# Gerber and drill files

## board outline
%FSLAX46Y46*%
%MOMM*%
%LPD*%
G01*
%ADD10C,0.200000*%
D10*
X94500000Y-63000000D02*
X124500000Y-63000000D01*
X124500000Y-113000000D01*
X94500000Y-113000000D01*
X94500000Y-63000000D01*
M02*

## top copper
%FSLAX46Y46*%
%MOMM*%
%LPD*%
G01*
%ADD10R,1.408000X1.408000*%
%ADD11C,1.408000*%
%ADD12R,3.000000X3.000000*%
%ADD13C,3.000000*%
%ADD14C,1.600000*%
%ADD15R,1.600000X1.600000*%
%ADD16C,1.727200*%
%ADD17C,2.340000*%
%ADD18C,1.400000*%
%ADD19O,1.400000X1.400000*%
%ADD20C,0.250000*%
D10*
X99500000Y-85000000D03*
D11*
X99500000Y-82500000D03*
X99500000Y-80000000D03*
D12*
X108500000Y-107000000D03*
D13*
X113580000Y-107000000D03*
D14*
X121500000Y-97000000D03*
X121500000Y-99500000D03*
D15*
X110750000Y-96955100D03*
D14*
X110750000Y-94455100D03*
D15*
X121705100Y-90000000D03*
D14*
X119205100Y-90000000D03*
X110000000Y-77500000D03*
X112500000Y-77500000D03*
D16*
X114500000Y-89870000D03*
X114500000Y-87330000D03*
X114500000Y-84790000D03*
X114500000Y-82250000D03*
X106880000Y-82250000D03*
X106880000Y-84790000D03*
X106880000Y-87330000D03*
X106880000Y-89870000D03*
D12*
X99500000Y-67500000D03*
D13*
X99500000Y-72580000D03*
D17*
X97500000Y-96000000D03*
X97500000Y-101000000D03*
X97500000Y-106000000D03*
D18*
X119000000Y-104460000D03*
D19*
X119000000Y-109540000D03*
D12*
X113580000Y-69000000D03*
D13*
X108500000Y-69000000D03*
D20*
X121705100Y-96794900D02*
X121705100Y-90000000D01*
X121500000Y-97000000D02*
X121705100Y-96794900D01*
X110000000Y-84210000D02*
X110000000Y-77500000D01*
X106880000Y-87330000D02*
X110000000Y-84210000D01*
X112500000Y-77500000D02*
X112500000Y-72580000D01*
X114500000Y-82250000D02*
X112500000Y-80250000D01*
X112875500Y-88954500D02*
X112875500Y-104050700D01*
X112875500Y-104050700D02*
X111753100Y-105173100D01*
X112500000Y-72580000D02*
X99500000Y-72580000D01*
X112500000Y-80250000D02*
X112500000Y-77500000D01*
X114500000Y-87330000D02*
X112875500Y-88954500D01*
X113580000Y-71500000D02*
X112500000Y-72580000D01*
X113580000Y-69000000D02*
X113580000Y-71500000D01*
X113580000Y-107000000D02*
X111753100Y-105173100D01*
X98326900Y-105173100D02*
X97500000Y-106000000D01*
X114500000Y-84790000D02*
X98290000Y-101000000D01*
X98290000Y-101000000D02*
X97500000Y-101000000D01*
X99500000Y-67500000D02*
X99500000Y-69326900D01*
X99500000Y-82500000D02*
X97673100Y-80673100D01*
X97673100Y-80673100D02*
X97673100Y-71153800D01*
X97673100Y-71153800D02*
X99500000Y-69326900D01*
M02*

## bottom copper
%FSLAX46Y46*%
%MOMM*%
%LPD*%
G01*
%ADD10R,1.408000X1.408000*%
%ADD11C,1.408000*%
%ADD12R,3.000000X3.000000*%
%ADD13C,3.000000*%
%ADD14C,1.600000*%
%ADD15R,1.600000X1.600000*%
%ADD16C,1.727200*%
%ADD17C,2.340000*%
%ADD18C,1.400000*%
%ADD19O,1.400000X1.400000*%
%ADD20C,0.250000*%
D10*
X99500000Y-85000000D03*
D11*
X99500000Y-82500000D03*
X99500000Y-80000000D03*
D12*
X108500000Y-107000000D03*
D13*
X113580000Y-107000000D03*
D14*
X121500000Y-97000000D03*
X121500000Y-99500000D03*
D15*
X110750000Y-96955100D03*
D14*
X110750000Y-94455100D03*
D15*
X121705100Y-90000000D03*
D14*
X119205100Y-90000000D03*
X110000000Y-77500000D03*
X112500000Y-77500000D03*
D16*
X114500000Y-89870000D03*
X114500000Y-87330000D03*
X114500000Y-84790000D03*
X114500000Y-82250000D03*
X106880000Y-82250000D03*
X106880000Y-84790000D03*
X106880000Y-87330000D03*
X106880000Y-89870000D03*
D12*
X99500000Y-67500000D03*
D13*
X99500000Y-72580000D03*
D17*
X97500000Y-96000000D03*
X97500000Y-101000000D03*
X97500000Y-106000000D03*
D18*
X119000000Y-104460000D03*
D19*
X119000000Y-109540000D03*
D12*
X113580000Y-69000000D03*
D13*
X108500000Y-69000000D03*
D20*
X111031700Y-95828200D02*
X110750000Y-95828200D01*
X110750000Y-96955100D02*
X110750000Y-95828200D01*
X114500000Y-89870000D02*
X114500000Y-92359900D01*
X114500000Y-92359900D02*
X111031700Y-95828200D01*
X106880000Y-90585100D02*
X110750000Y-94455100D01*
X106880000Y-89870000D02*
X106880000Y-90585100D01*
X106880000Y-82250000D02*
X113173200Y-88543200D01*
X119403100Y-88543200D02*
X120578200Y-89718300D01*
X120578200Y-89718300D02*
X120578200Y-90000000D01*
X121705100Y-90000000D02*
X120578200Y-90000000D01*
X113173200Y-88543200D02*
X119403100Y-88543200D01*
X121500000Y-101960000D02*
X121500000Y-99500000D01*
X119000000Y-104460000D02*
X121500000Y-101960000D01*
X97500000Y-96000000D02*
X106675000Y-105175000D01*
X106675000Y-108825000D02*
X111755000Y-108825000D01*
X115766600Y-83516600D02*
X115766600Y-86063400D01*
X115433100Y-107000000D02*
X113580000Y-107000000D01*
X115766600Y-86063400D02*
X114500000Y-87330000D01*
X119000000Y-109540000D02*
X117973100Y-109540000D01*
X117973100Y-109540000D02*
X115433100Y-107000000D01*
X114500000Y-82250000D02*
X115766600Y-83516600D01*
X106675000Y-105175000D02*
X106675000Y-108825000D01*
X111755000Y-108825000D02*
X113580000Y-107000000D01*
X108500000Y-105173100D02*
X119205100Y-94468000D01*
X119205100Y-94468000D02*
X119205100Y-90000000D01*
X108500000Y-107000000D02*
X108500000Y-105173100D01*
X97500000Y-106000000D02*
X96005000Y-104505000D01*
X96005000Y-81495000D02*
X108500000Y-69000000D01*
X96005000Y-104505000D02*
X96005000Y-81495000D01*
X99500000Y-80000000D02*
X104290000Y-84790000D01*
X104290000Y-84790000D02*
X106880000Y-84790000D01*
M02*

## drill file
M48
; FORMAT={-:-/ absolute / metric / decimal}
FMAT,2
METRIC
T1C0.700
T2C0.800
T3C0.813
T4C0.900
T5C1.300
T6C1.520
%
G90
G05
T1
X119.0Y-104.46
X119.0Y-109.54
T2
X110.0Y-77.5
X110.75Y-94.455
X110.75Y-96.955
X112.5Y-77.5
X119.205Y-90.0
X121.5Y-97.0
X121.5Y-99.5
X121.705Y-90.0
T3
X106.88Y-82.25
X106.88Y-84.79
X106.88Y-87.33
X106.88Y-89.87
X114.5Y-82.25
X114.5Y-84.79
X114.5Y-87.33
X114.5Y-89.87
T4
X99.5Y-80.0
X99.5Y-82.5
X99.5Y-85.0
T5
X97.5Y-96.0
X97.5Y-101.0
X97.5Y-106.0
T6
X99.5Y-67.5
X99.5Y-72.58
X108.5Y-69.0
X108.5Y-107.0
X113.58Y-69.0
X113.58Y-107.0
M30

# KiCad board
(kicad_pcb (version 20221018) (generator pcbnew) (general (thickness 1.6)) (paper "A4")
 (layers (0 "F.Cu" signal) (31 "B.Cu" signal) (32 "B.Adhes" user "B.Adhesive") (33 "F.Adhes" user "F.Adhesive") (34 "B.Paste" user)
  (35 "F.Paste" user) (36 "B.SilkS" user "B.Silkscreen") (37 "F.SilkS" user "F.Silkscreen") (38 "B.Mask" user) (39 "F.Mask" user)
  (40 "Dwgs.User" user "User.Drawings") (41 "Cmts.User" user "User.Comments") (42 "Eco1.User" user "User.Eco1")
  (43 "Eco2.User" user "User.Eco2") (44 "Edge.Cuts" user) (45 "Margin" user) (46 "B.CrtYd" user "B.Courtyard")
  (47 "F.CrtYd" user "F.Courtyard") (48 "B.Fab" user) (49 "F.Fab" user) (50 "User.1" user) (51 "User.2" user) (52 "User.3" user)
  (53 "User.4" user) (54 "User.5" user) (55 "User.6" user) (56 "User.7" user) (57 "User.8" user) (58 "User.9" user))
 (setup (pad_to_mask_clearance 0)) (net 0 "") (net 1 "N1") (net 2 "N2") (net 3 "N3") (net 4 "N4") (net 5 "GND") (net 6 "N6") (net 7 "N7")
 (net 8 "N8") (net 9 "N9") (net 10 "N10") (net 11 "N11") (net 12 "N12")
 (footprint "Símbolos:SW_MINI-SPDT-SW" (layer "F.Cu") (at 99.5 82.5 90)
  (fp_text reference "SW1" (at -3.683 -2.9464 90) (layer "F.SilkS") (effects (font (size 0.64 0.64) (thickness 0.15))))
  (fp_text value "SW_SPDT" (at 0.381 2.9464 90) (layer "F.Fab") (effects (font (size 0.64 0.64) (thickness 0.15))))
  (pad "1" thru_hole rect (at -2.5 0 90) (size 1.408 1.408) (drill 0.9) (layers "*.Cu" "*.Mask") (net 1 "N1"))
  (pad "2" thru_hole circle (at 0 0 90) (size 1.408 1.408) (drill 0.9) (layers "*.Cu" "*.Mask") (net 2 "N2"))
  (pad "3" thru_hole circle (at 2.5 0 90) (size 1.408 1.408) (drill 0.9) (layers "*.Cu" "*.Mask") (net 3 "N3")))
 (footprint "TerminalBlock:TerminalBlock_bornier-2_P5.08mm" (layer "F.Cu") (at 108.5 107)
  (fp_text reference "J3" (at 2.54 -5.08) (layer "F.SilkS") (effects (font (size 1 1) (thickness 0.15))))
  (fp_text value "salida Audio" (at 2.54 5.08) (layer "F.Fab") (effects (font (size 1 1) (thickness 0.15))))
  (pad "1" thru_hole rect (at 0 0) (size 3 3) (drill 1.52) (layers "*.Cu" "*.Mask") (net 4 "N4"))
  (pad "2" thru_hole circle (at 5.08 0) (size 3 3) (drill 1.52) (layers "*.Cu" "*.Mask") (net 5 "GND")))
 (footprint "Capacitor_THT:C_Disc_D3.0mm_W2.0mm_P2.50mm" (layer "F.Cu") (at 121.5 97 -90)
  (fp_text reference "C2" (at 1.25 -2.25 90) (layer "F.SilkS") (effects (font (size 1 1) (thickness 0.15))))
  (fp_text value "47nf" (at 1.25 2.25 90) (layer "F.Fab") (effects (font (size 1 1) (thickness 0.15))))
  (pad "1" thru_hole circle (at 0 0 270) (size 1.6 1.6) (drill 0.8) (layers "*.Cu" "*.Mask") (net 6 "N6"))
  (pad "2" thru_hole circle (at 2.5 0 270) (size 1.6 1.6) (drill 0.8) (layers "*.Cu" "*.Mask") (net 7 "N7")))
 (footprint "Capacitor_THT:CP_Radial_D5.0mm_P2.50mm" (layer "F.Cu") (at 110.75 96.9551 90)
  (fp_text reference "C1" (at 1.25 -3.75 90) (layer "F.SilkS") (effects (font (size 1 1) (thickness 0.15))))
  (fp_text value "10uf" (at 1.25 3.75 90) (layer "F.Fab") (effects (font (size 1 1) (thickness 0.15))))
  (pad "1" thru_hole rect (at 0 0 90) (size 1.6 1.6) (drill 0.8) (layers "*.Cu" "*.Mask") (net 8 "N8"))
  (pad "2" thru_hole circle (at 2.5 0 90) (size 1.6 1.6) (drill 0.8) (layers "*.Cu" "*.Mask") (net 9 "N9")))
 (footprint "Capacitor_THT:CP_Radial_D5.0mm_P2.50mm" (layer "F.Cu") (at 121.7051 90 180)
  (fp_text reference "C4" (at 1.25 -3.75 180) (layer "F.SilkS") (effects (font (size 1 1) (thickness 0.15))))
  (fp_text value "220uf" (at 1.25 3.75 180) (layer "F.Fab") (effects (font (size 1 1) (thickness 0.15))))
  (pad "1" thru_hole rect (at 0 0 180) (size 1.6 1.6) (drill 0.8) (layers "*.Cu" "*.Mask") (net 6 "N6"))
  (pad "2" thru_hole circle (at 2.5 0 180) (size 1.6 1.6) (drill 0.8) (layers "*.Cu" "*.Mask") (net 4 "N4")))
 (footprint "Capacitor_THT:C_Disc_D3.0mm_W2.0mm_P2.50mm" (layer "F.Cu") (at 110 77.5)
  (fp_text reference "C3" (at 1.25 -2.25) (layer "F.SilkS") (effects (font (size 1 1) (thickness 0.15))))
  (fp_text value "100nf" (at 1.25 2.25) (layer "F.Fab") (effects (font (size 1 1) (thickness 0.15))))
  (pad "1" thru_hole circle (at 0 0) (size 1.6 1.6) (drill 0.8) (layers "*.Cu" "*.Mask") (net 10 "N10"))
  (pad "2" thru_hole circle (at 2.5 0) (size 1.6 1.6) (drill 0.8) (layers "*.Cu" "*.Mask") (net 5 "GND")))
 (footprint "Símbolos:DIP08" (layer "F.Cu") (at 110.69 86.06 90)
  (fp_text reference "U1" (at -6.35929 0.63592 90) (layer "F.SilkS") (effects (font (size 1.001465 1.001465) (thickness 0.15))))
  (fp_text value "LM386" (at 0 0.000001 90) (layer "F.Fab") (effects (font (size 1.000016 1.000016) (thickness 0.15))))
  (pad "1" thru_hole circle (at -3.81 3.81 90) (size 1.7272 1.7272) (drill 0.8128) (layers "*.Cu" "*.Mask") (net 8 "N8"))
  (pad "2" thru_hole circle (at -1.27 3.81 90) (size 1.7272 1.7272) (drill 0.8128) (layers "*.Cu" "*.Mask") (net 5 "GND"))
  (pad "3" thru_hole circle (at 1.27 3.81 90) (size 1.7272 1.7272) (drill 0.8128) (layers "*.Cu" "*.Mask") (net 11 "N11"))
  (pad "4" thru_hole circle (at 3.81 3.81 90) (size 1.7272 1.7272) (drill 0.8128) (layers "*.Cu" "*.Mask") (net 5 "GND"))
  (pad "5" thru_hole circle (at 3.81 -3.81 90) (size 1.7272 1.7272) (drill 0.8128) (layers "*.Cu" "*.Mask") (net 6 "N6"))
  (pad "6" thru_hole circle (at 1.27 -3.81 90) (size 1.7272 1.7272) (drill 0.8128) (layers "*.Cu" "*.Mask") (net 3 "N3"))
  (pad "7" thru_hole circle (at -1.27 -3.81 90) (size 1.7272 1.7272) (drill 0.8128) (layers "*.Cu" "*.Mask") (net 10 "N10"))
  (pad "8" thru_hole circle (at -3.81 -3.81 90) (size 1.7272 1.7272) (drill 0.8128) (layers "*.Cu" "*.Mask") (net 9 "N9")))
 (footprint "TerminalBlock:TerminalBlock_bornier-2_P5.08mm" (layer "F.Cu") (at 99.5 67.5 -90)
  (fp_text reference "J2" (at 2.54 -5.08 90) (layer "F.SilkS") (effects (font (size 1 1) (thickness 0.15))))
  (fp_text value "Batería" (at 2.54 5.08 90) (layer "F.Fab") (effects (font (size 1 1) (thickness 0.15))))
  (pad "1" thru_hole rect (at 0 0 270) (size 3 3) (drill 1.52) (layers "*.Cu" "*.Mask") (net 2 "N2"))
  (pad "2" thru_hole circle (at 5.08 0 270) (size 3 3) (drill 1.52) (layers "*.Cu" "*.Mask") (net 5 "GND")))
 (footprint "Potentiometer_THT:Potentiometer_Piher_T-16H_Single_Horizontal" (layer "F.Cu") (at 97.5 96 180)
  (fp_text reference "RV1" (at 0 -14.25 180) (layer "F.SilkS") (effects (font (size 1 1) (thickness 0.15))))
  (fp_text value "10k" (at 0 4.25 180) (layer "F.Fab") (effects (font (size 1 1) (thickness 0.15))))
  (pad "1" thru_hole circle (at 0 0 180) (size 2.34 2.34) (drill 1.3) (layers "*.Cu" "*.Mask") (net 5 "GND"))
  (pad "2" thru_hole circle (at 0 -5 180) (size 2.34 2.34) (drill 1.3) (layers "*.Cu" "*.Mask") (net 11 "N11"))
  (pad "3" thru_hole circle (at 0 -10 180) (size 2.34 2.34) (drill 1.3) (layers "*.Cu" "*.Mask") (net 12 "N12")))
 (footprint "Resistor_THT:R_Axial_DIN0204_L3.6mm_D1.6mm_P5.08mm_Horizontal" (layer "F.Cu") (at 119 104.46 -90)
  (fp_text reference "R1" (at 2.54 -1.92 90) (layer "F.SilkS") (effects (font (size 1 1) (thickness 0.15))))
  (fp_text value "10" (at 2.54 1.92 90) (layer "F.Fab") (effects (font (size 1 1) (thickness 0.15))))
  (pad "1" thru_hole circle (at 0 0 270) (size 1.4 1.4) (drill 0.7) (layers "*.Cu" "*.Mask") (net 7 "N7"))
  (pad "2" thru_hole oval (at 5.08 0 270) (size 1.4 1.4) (drill 0.7) (layers "*.Cu" "*.Mask") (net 5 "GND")))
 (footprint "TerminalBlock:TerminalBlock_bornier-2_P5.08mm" (layer "F.Cu") (at 113.58 69 180)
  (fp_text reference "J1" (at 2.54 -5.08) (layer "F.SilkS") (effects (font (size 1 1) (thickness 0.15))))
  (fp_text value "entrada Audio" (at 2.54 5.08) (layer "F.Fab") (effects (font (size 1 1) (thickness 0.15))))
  (pad "1" thru_hole rect (at 0 0 180) (size 3 3) (drill 1.52) (layers "*.Cu" "*.Mask") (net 5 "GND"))
  (pad "2" thru_hole circle (at 5.08 0 180) (size 3 3) (drill 1.52) (layers "*.Cu" "*.Mask") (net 12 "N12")))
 (gr_rect (start 94.5 63) (end 124.5 113) (stroke (width 0.2) (type default)) (fill none) (layer "Edge.Cuts"))
 (segment (start 111.0317 95.8282) (end 110.75 95.8282) (width 0.25) (layer "B.Cu") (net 8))
 (segment (start 110.75 96.9551) (end 110.75 95.8282) (width 0.25) (layer "B.Cu") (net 8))
 (segment (start 114.5 89.87) (end 114.5 92.3599) (width 0.25) (layer "B.Cu") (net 8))
 (segment (start 114.5 92.3599) (end 111.0317 95.8282) (width 0.25) (layer "B.Cu") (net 8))
 (segment (start 106.88 90.5851) (end 110.75 94.4551) (width 0.25) (layer "B.Cu") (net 9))
 (segment (start 106.88 89.87) (end 106.88 90.5851) (width 0.25) (layer "B.Cu") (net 9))
 (segment (start 121.7051 96.7949) (end 121.7051 90) (width 0.25) (layer "F.Cu") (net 6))
 (segment (start 121.5 97) (end 121.7051 96.7949) (width 0.25) (layer "F.Cu") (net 6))
 (segment (start 106.88 82.25) (end 113.1732 88.5432) (width 0.25) (layer "B.Cu") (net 6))
 (segment (start 119.4031 88.5432) (end 120.5782 89.7183) (width 0.25) (layer "B.Cu") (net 6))
 (segment (start 120.5782 89.7183) (end 120.5782 90) (width 0.25) (layer "B.Cu") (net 6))
 (segment (start 121.7051 90) (end 120.5782 90) (width 0.25) (layer "B.Cu") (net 6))
 (segment (start 113.1732 88.5432) (end 119.4031 88.5432) (width 0.25) (layer "B.Cu") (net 6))
 (segment (start 121.5 101.96) (end 121.5 99.5) (width 0.25) (layer "B.Cu") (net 7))
 (segment (start 119 104.46) (end 121.5 101.96) (width 0.25) (layer "B.Cu") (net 7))
 (segment (start 110 84.21) (end 110 77.5) (width 0.25) (layer "F.Cu") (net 10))
 (segment (start 106.88 87.33) (end 110 84.21) (width 0.25) (layer "F.Cu") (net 10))
 (segment (start 112.5 77.5) (end 112.5 72.58) (width 0.25) (layer "F.Cu") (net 5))
 (segment (start 114.5 82.25) (end 112.5 80.25) (width 0.25) (layer "F.Cu") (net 5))
 (segment (start 112.8755 88.9545) (end 112.8755 104.0507) (width 0.25) (layer "F.Cu") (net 5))
 (segment (start 112.8755 104.0507) (end 111.7531 105.1731) (width 0.25) (layer "F.Cu") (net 5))
 (segment (start 112.5 72.58) (end 99.5 72.58) (width 0.25) (layer "F.Cu") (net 5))
 (segment (start 112.5 80.25) (end 112.5 77.5) (width 0.25) (layer "F.Cu") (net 5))
 (segment (start 114.5 87.33) (end 112.8755 88.9545) (width 0.25) (layer "F.Cu") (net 5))
 (segment (start 113.58 71.5) (end 112.5 72.58) (width 0.25) (layer "F.Cu") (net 5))
 (segment (start 113.58 69) (end 113.58 71.5) (width 0.25) (layer "F.Cu") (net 5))
 (segment (start 113.58 107) (end 111.7531 105.1731) (width 0.25) (layer "F.Cu") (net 5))
 (segment (start 97.5 96) (end 106.675 105.175) (width 0.25) (layer "B.Cu") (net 5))
 (segment (start 106.675 108.825) (end 111.755 108.825) (width 0.25) (layer "B.Cu") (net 5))
 (segment (start 115.7666 83.5166) (end 115.7666 86.0634) (width 0.25) (layer "B.Cu") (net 5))
 (segment (start 115.4331 107) (end 113.58 107) (width 0.25) (layer "B.Cu") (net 5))
 (segment (start 115.7666 86.0634) (end 114.5 87.33) (width 0.25) (layer "B.Cu") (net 5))
 (segment (start 119 109.54) (end 117.9731 109.54) (width 0.25) (layer "B.Cu") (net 5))
 (segment (start 117.9731 109.54) (end 115.4331 107) (width 0.25) (layer "B.Cu") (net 5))
 (segment (start 114.5 82.25) (end 115.7666 83.5166) (width 0.25) (layer "B.Cu") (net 5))
 (segment (start 106.675 105.175) (end 106.675 108.825) (width 0.25) (layer "B.Cu") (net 5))
 (segment (start 111.755 108.825) (end 113.58 107) (width 0.25) (layer "B.Cu") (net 5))
 (segment (start 108.5 105.1731) (end 119.2051 94.468) (width 0.25) (layer "B.Cu") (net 4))
 (segment (start 119.2051 94.468) (end 119.2051 90) (width 0.25) (layer "B.Cu") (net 4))
 (segment (start 108.5 107) (end 108.5 105.1731) (width 0.25) (layer "B.Cu") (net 4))
 (segment (start 98.3269 105.1731) (end 97.5 106) (width 0.25) (layer "F.Cu") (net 12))
 (segment (start 97.5 106) (end 96.005 104.505) (width 0.25) (layer "B.Cu") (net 12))
 (segment (start 96.005 81.495) (end 108.5 69) (width 0.25) (layer "B.Cu") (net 12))
 (segment (start 96.005 104.505) (end 96.005 81.495) (width 0.25) (layer "B.Cu") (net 12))
 (segment (start 114.5 84.79) (end 98.29 101) (width 0.25) (layer "F.Cu") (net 11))
 (segment (start 98.29 101) (end 97.5 101) (width 0.25) (layer "F.Cu") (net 11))
 (segment (start 99.5 80) (end 104.29 84.79) (width 0.25) (layer "B.Cu") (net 3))
 (segment (start 104.29 84.79) (end 106.88 84.79) (width 0.25) (layer "B.Cu") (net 3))
 (segment (start 99.5 67.5) (end 99.5 69.3269) (width 0.25) (layer "F.Cu") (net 2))
 (segment (start 99.5 82.5) (end 97.6731 80.6731) (width 0.25) (layer "F.Cu") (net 2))
 (segment (start 97.6731 80.6731) (end 97.6731 71.1538) (width 0.25) (layer "F.Cu") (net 2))
 (segment (start 97.6731 71.1538) (end 99.5 69.3269) (width 0.25) (layer "F.Cu") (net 2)))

